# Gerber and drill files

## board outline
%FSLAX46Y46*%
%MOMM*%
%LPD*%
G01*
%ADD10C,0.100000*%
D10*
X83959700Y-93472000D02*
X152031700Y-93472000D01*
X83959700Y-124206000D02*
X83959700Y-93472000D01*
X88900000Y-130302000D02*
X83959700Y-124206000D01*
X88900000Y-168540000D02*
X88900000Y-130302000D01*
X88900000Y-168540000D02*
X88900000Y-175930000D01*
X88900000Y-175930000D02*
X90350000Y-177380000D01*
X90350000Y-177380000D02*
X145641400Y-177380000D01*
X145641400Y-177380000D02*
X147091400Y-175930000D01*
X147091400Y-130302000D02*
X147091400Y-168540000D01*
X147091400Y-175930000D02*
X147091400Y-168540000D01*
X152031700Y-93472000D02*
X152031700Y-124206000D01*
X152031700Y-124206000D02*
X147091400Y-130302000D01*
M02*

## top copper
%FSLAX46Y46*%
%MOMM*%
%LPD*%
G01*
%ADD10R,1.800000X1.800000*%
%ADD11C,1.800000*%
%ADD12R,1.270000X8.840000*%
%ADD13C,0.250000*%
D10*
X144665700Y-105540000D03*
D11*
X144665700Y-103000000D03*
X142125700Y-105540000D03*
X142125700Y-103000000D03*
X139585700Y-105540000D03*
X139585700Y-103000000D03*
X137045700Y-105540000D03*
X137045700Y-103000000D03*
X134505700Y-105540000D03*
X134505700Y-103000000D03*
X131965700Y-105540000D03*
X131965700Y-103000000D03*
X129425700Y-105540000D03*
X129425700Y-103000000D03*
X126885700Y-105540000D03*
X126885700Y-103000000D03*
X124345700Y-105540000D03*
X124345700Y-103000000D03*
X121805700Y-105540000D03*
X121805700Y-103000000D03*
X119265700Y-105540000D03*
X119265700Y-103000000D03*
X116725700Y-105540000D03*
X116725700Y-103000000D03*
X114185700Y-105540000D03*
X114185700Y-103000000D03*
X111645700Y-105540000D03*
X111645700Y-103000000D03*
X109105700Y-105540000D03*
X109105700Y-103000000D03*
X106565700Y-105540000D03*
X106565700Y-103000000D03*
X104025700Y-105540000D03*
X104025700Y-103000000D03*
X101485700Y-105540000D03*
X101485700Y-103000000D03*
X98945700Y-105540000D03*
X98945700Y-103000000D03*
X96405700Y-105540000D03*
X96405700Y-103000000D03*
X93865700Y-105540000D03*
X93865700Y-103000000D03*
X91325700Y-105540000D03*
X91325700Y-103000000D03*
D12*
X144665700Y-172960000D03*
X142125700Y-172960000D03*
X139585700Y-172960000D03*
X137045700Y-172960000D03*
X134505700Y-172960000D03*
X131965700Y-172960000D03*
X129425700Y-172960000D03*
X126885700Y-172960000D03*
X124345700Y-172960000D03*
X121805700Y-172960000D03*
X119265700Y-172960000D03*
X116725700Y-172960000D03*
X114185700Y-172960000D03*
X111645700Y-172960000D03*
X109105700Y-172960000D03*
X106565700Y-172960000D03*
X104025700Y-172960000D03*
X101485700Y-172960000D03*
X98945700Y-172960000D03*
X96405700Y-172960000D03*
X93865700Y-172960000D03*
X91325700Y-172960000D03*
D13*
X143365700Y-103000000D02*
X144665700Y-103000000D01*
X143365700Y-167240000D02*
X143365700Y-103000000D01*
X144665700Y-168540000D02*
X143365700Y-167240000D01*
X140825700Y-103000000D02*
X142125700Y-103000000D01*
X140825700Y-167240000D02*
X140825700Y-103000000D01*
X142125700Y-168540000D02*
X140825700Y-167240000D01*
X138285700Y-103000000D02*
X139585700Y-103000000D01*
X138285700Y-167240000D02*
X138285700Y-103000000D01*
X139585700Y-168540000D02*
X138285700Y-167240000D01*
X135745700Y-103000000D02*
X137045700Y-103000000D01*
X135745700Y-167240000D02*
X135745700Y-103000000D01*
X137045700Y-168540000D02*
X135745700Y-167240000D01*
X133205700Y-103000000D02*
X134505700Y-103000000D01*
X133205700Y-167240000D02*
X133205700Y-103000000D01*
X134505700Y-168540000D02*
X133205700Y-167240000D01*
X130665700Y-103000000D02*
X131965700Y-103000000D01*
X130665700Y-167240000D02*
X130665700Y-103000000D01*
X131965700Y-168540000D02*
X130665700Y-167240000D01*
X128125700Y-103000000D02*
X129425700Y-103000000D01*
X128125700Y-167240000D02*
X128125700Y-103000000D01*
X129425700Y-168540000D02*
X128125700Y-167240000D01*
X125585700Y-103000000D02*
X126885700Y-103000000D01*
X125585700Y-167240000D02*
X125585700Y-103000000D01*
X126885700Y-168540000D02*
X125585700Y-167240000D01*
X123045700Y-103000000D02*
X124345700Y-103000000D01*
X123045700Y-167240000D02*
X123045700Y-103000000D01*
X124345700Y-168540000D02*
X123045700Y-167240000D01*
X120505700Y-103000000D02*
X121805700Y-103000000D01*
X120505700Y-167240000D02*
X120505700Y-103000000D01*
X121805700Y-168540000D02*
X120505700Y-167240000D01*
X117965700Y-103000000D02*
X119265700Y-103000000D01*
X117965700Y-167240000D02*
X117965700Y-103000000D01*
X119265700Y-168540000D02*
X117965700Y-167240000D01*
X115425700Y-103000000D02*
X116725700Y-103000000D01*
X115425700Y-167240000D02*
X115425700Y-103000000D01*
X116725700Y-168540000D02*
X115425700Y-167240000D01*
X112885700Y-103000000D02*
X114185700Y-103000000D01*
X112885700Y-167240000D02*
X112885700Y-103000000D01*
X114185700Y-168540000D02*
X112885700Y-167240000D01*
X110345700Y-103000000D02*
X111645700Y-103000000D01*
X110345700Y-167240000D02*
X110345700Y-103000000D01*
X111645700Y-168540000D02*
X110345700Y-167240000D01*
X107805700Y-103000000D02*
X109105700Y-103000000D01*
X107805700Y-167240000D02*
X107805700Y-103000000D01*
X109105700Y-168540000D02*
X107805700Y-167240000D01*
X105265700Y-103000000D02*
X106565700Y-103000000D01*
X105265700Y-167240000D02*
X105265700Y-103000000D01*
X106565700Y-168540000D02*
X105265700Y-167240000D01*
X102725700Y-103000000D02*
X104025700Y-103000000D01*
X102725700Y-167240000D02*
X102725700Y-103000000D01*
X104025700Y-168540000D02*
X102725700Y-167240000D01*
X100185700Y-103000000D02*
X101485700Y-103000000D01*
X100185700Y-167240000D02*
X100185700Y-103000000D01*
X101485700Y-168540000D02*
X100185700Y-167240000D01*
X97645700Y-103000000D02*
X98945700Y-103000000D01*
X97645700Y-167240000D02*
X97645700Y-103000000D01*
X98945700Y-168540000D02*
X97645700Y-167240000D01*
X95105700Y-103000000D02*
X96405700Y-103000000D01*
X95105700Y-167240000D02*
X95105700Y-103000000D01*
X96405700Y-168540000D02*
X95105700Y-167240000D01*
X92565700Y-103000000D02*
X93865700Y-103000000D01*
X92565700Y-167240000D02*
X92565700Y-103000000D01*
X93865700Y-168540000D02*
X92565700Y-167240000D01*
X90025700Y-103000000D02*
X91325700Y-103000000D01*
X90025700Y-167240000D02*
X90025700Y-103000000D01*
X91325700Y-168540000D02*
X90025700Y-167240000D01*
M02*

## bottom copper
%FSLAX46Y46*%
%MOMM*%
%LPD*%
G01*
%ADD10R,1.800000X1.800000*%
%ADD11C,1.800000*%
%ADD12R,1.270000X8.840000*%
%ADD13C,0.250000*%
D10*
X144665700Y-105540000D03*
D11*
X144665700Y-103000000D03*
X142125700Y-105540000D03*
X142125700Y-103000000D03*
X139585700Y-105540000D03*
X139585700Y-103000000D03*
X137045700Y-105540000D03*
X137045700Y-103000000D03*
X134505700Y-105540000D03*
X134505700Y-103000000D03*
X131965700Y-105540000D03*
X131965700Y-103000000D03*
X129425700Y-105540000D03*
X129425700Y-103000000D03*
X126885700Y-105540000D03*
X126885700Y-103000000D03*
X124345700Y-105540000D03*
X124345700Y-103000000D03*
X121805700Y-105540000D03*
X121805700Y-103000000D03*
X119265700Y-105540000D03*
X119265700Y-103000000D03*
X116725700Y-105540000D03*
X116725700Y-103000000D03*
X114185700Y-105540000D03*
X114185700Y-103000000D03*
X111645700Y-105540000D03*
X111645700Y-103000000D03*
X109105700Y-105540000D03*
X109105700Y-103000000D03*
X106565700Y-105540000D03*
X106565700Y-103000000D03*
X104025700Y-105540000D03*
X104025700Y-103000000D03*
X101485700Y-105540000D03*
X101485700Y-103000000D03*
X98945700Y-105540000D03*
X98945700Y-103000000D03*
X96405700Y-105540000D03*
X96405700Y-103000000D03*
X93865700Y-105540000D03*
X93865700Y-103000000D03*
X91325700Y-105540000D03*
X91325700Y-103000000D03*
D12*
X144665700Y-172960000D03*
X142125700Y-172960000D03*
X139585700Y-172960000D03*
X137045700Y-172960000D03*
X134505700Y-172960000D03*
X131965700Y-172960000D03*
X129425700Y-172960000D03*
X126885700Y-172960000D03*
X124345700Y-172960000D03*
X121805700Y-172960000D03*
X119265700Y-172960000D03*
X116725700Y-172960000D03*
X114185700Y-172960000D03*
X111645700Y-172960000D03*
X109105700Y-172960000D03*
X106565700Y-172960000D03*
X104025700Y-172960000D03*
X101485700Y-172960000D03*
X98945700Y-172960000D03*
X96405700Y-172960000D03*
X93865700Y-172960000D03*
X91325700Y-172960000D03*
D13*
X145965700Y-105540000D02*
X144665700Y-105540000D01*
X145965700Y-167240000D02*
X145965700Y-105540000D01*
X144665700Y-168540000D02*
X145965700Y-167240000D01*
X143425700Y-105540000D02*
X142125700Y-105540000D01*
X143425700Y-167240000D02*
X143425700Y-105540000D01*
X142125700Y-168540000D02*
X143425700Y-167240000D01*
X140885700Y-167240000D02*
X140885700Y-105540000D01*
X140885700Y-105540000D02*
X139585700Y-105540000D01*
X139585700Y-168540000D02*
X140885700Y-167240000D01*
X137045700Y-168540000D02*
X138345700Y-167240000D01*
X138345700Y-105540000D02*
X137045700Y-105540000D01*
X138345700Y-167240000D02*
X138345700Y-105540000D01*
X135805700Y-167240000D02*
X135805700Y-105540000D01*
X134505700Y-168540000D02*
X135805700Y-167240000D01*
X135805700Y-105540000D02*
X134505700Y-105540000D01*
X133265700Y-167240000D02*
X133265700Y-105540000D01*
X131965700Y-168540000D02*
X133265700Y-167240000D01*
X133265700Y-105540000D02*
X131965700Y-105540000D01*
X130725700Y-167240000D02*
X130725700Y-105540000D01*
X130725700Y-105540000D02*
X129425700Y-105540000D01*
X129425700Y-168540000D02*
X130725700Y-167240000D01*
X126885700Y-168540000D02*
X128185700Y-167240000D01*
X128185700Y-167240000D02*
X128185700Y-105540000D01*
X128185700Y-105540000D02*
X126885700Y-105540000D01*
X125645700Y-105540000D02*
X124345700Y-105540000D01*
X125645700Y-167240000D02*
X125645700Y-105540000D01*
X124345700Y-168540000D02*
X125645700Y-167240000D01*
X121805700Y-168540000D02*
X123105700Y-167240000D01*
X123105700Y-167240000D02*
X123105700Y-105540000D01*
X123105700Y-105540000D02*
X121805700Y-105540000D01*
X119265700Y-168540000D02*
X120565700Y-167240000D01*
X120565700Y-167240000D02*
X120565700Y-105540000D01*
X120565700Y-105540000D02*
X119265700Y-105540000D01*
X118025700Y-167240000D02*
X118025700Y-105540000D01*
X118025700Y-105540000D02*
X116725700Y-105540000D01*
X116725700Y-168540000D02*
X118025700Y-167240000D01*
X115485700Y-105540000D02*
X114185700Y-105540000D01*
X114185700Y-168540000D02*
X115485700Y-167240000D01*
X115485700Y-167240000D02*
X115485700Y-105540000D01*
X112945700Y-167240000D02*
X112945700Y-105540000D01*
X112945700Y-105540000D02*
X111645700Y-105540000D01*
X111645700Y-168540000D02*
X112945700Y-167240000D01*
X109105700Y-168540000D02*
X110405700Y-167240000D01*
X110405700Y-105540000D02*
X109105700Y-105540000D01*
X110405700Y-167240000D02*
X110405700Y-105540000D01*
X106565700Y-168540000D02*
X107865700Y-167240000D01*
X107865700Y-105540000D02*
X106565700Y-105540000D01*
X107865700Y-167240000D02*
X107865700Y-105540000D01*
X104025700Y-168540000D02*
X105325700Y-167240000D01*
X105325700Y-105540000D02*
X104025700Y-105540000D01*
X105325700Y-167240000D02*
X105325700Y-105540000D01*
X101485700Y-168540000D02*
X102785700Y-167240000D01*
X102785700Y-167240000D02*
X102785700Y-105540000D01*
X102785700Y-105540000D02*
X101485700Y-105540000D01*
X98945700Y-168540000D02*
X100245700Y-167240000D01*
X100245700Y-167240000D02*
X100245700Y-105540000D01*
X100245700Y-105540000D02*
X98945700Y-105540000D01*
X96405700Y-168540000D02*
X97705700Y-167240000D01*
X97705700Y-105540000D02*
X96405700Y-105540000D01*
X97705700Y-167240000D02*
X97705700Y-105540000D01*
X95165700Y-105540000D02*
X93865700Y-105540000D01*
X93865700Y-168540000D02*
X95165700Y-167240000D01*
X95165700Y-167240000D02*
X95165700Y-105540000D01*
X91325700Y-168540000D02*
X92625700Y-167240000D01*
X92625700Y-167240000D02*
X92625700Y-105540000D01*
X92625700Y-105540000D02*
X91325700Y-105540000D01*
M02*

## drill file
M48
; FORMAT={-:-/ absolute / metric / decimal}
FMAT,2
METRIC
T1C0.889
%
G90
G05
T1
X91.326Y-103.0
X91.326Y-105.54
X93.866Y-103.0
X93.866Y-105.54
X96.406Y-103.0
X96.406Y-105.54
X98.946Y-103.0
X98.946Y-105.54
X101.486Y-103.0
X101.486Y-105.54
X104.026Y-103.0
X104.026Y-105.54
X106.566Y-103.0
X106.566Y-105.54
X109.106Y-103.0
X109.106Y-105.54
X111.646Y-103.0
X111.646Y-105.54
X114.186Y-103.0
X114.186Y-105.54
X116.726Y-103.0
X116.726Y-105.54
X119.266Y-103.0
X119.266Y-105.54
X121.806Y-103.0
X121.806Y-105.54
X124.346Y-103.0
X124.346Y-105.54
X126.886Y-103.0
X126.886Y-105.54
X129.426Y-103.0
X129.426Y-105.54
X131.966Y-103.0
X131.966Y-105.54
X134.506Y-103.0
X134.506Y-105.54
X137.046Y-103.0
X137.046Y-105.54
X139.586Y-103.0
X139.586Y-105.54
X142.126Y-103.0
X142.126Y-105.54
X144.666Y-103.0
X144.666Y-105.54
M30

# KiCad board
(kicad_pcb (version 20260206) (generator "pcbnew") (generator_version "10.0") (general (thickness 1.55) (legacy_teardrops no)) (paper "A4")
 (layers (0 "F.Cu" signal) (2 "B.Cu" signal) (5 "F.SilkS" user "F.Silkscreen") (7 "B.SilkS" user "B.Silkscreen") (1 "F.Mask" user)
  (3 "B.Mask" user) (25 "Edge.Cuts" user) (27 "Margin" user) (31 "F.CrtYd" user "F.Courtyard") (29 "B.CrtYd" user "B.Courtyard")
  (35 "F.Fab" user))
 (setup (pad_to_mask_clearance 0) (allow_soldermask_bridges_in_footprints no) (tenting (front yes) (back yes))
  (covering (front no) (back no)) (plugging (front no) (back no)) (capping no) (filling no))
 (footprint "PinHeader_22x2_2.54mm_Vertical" (layer "F.Cu") (at 0 0)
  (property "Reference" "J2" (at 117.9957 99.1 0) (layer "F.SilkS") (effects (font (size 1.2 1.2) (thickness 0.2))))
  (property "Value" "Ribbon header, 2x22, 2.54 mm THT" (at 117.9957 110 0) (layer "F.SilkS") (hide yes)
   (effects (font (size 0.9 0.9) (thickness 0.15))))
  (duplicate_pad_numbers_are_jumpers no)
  (pad "1" thru_hole rect (at 144.6657 105.54) (size 1.8 1.8) (drill 0.889) (layers "*.Cu" "*.Mask") (remove_unused_layers no)
   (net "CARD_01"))
  (pad "2" thru_hole circle (at 144.6657 103) (size 1.8 1.8) (drill 0.889) (layers "*.Cu" "*.Mask") (remove_unused_layers no)
   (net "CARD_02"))
  (pad "3" thru_hole circle (at 142.1257 105.54) (size 1.8 1.8) (drill 0.889) (layers "*.Cu" "*.Mask") (remove_unused_layers no)
   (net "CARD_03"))
  (pad "4" thru_hole circle (at 142.1257 103) (size 1.8 1.8) (drill 0.889) (layers "*.Cu" "*.Mask") (remove_unused_layers no)
   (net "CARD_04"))
  (pad "5" thru_hole circle (at 139.5857 105.54) (size 1.8 1.8) (drill 0.889) (layers "*.Cu" "*.Mask") (remove_unused_layers no)
   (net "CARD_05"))
  (pad "6" thru_hole circle (at 139.5857 103) (size 1.8 1.8) (drill 0.889) (layers "*.Cu" "*.Mask") (remove_unused_layers no)
   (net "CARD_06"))
  (pad "7" thru_hole circle (at 137.0457 105.54) (size 1.8 1.8) (drill 0.889) (layers "*.Cu" "*.Mask") (remove_unused_layers no)
   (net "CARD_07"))
  (pad "8" thru_hole circle (at 137.0457 103) (size 1.8 1.8) (drill 0.889) (layers "*.Cu" "*.Mask") (remove_unused_layers no)
   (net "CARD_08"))
  (pad "9" thru_hole circle (at 134.5057 105.54) (size 1.8 1.8) (drill 0.889) (layers "*.Cu" "*.Mask") (remove_unused_layers no)
   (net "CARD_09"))
  (pad "10" thru_hole circle (at 134.5057 103) (size 1.8 1.8) (drill 0.889) (layers "*.Cu" "*.Mask") (remove_unused_layers no)
   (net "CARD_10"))
  (pad "11" thru_hole circle (at 131.9657 105.54) (size 1.8 1.8) (drill 0.889) (layers "*.Cu" "*.Mask") (remove_unused_layers no)
   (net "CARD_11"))
  (pad "12" thru_hole circle (at 131.9657 103) (size 1.8 1.8) (drill 0.889) (layers "*.Cu" "*.Mask") (remove_unused_layers no)
   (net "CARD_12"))
  (pad "13" thru_hole circle (at 129.4257 105.54) (size 1.8 1.8) (drill 0.889) (layers "*.Cu" "*.Mask") (remove_unused_layers no)
   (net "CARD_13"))
  (pad "14" thru_hole circle (at 129.4257 103) (size 1.8 1.8) (drill 0.889) (layers "*.Cu" "*.Mask") (remove_unused_layers no)
   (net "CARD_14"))
  (pad "15" thru_hole circle (at 126.8857 105.54) (size 1.8 1.8) (drill 0.889) (layers "*.Cu" "*.Mask") (remove_unused_layers no)
   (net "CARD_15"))
  (pad "16" thru_hole circle (at 126.8857 103) (size 1.8 1.8) (drill 0.889) (layers "*.Cu" "*.Mask") (remove_unused_layers no)
   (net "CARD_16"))
  (pad "17" thru_hole circle (at 124.3457 105.54) (size 1.8 1.8) (drill 0.889) (layers "*.Cu" "*.Mask") (remove_unused_layers no)
   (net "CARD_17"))
  (pad "18" thru_hole circle (at 124.3457 103) (size 1.8 1.8) (drill 0.889) (layers "*.Cu" "*.Mask") (remove_unused_layers no)
   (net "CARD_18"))
  (pad "19" thru_hole circle (at 121.8057 105.54) (size 1.8 1.8) (drill 0.889) (layers "*.Cu" "*.Mask") (remove_unused_layers no)
   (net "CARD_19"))
  (pad "20" thru_hole circle (at 121.8057 103) (size 1.8 1.8) (drill 0.889) (layers "*.Cu" "*.Mask") (remove_unused_layers no)
   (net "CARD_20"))
  (pad "21" thru_hole circle (at 119.2657 105.54) (size 1.8 1.8) (drill 0.889) (layers "*.Cu" "*.Mask") (remove_unused_layers no)
   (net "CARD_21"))
  (pad "22" thru_hole circle (at 119.2657 103) (size 1.8 1.8) (drill 0.889) (layers "*.Cu" "*.Mask") (remove_unused_layers no)
   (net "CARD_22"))
  (pad "23" thru_hole circle (at 116.7257 105.54) (size 1.8 1.8) (drill 0.889) (layers "*.Cu" "*.Mask") (remove_unused_layers no)
   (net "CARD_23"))
  (pad "24" thru_hole circle (at 116.7257 103) (size 1.8 1.8) (drill 0.889) (layers "*.Cu" "*.Mask") (remove_unused_layers no)
   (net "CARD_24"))
  (pad "25" thru_hole circle (at 114.1857 105.54) (size 1.8 1.8) (drill 0.889) (layers "*.Cu" "*.Mask") (remove_unused_layers no)
   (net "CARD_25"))
  (pad "26" thru_hole circle (at 114.1857 103) (size 1.8 1.8) (drill 0.889) (layers "*.Cu" "*.Mask") (remove_unused_layers no)
   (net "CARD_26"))
  (pad "27" thru_hole circle (at 111.6457 105.54) (size 1.8 1.8) (drill 0.889) (layers "*.Cu" "*.Mask") (remove_unused_layers no)
   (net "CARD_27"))
  (pad "28" thru_hole circle (at 111.6457 103) (size 1.8 1.8) (drill 0.889) (layers "*.Cu" "*.Mask") (remove_unused_layers no)
   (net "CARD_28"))
  (pad "29" thru_hole circle (at 109.1057 105.54) (size 1.8 1.8) (drill 0.889) (layers "*.Cu" "*.Mask") (remove_unused_layers no)
   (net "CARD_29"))
  (pad "30" thru_hole circle (at 109.1057 103) (size 1.8 1.8) (drill 0.889) (layers "*.Cu" "*.Mask") (remove_unused_layers no)
   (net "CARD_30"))
  (pad "31" thru_hole circle (at 106.5657 105.54) (size 1.8 1.8) (drill 0.889) (layers "*.Cu" "*.Mask") (remove_unused_layers no)
   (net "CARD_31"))
  (pad "32" thru_hole circle (at 106.5657 103) (size 1.8 1.8) (drill 0.889) (layers "*.Cu" "*.Mask") (remove_unused_layers no)
   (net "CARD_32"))
  (pad "33" thru_hole circle (at 104.0257 105.54) (size 1.8 1.8) (drill 0.889) (layers "*.Cu" "*.Mask") (remove_unused_layers no)
   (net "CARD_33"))
  (pad "34" thru_hole circle (at 104.0257 103) (size 1.8 1.8) (drill 0.889) (layers "*.Cu" "*.Mask") (remove_unused_layers no)
   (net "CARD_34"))
  (pad "35" thru_hole circle (at 101.4857 105.54) (size 1.8 1.8) (drill 0.889) (layers "*.Cu" "*.Mask") (remove_unused_layers no)
   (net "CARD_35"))
  (pad "36" thru_hole circle (at 101.4857 103) (size 1.8 1.8) (drill 0.889) (layers "*.Cu" "*.Mask") (remove_unused_layers no)
   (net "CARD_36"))
  (pad "37" thru_hole circle (at 98.9457 105.54) (size 1.8 1.8) (drill 0.889) (layers "*.Cu" "*.Mask") (remove_unused_layers no)
   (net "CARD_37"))
  (pad "38" thru_hole circle (at 98.9457 103) (size 1.8 1.8) (drill 0.889) (layers "*.Cu" "*.Mask") (remove_unused_layers no)
   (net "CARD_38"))
  (pad "39" thru_hole circle (at 96.4057 105.54) (size 1.8 1.8) (drill 0.889) (layers "*.Cu" "*.Mask") (remove_unused_layers no)
   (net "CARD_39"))
  (pad "40" thru_hole circle (at 96.4057 103) (size 1.8 1.8) (drill 0.889) (layers "*.Cu" "*.Mask") (remove_unused_layers no)
   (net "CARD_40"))
  (pad "41" thru_hole circle (at 93.8657 105.54) (size 1.8 1.8) (drill 0.889) (layers "*.Cu" "*.Mask") (remove_unused_layers no)
   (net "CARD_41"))
  (pad "42" thru_hole circle (at 93.8657 103) (size 1.8 1.8) (drill 0.889) (layers "*.Cu" "*.Mask") (remove_unused_layers no)
   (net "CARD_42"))
  (pad "43" thru_hole circle (at 91.3257 105.54) (size 1.8 1.8) (drill 0.889) (layers "*.Cu" "*.Mask") (remove_unused_layers no)
   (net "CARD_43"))
  (pad "44" thru_hole circle (at 91.3257 103) (size 1.8 1.8) (drill 0.889) (layers "*.Cu" "*.Mask") (remove_unused_layers no)
   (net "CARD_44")))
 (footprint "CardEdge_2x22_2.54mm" (layer "F.Cu") (at 0 -15)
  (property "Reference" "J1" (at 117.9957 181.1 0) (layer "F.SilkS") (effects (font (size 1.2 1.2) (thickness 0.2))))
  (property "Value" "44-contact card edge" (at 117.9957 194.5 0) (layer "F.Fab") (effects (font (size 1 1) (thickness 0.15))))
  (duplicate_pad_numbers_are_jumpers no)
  (pad "1" connect rect (at 144.6657 187.96) (size 1.27 8.84) (layers "B.Cu" "B.Mask") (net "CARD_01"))
  (pad "2" connect rect (at 144.6657 187.96) (size 1.27 8.84) (layers "F.Cu" "F.Mask") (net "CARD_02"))
  (pad "3" connect rect (at 142.1257 187.96) (size 1.27 8.84) (layers "B.Cu" "B.Mask") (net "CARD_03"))
  (pad "4" connect rect (at 142.1257 187.96) (size 1.27 8.84) (layers "F.Cu" "F.Mask") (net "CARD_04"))
  (pad "5" connect rect (at 139.5857 187.96) (size 1.27 8.84) (layers "B.Cu" "B.Mask") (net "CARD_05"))
  (pad "6" connect rect (at 139.5857 187.96) (size 1.27 8.84) (layers "F.Cu" "F.Mask") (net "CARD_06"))
  (pad "7" connect rect (at 137.0457 187.96) (size 1.27 8.84) (layers "B.Cu" "B.Mask") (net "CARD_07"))
  (pad "8" connect rect (at 137.0457 187.96) (size 1.27 8.84) (layers "F.Cu" "F.Mask") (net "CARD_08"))
  (pad "9" connect rect (at 134.5057 187.96) (size 1.27 8.84) (layers "B.Cu" "B.Mask") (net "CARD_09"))
  (pad "10" connect rect (at 134.5057 187.96) (size 1.27 8.84) (layers "F.Cu" "F.Mask") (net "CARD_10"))
  (pad "11" connect rect (at 131.9657 187.96) (size 1.27 8.84) (layers "B.Cu" "B.Mask") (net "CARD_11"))
  (pad "12" connect rect (at 131.9657 187.96) (size 1.27 8.84) (layers "F.Cu" "F.Mask") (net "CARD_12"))
  (pad "13" connect rect (at 129.4257 187.96) (size 1.27 8.84) (layers "B.Cu" "B.Mask") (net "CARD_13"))
  (pad "14" connect rect (at 129.4257 187.96) (size 1.27 8.84) (layers "F.Cu" "F.Mask") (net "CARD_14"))
  (pad "15" connect rect (at 126.8857 187.96) (size 1.27 8.84) (layers "B.Cu" "B.Mask") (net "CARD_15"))
  (pad "16" connect rect (at 126.8857 187.96) (size 1.27 8.84) (layers "F.Cu" "F.Mask") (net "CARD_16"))
  (pad "17" connect rect (at 124.3457 187.96) (size 1.27 8.84) (layers "B.Cu" "B.Mask") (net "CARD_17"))
  (pad "18" connect rect (at 124.3457 187.96) (size 1.27 8.84) (layers "F.Cu" "F.Mask") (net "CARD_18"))
  (pad "19" connect rect (at 121.8057 187.96) (size 1.27 8.84) (layers "B.Cu" "B.Mask") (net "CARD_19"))
  (pad "20" connect rect (at 121.8057 187.96) (size 1.27 8.84) (layers "F.Cu" "F.Mask") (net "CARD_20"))
  (pad "21" connect rect (at 119.2657 187.96) (size 1.27 8.84) (layers "B.Cu" "B.Mask") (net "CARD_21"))
  (pad "22" connect rect (at 119.2657 187.96) (size 1.27 8.84) (layers "F.Cu" "F.Mask") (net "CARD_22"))
  (pad "23" connect rect (at 116.7257 187.96) (size 1.27 8.84) (layers "B.Cu" "B.Mask") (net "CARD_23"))
  (pad "24" connect rect (at 116.7257 187.96) (size 1.27 8.84) (layers "F.Cu" "F.Mask") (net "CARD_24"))
  (pad "25" connect rect (at 114.1857 187.96) (size 1.27 8.84) (layers "B.Cu" "B.Mask") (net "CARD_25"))
  (pad "26" connect rect (at 114.1857 187.96) (size 1.27 8.84) (layers "F.Cu" "F.Mask") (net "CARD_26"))
  (pad "27" connect rect (at 111.6457 187.96) (size 1.27 8.84) (layers "B.Cu" "B.Mask") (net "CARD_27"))
  (pad "28" connect rect (at 111.6457 187.96) (size 1.27 8.84) (layers "F.Cu" "F.Mask") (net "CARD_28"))
  (pad "29" connect rect (at 109.1057 187.96) (size 1.27 8.84) (layers "B.Cu" "B.Mask") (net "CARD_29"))
  (pad "30" connect rect (at 109.1057 187.96) (size 1.27 8.84) (layers "F.Cu" "F.Mask") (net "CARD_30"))
  (pad "31" connect rect (at 106.5657 187.96) (size 1.27 8.84) (layers "B.Cu" "B.Mask") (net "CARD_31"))
  (pad "32" connect rect (at 106.5657 187.96) (size 1.27 8.84) (layers "F.Cu" "F.Mask") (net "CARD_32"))
  (pad "33" connect rect (at 104.0257 187.96) (size 1.27 8.84) (layers "B.Cu" "B.Mask") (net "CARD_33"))
  (pad "34" connect rect (at 104.0257 187.96) (size 1.27 8.84) (layers "F.Cu" "F.Mask") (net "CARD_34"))
  (pad "35" connect rect (at 101.4857 187.96) (size 1.27 8.84) (layers "B.Cu" "B.Mask") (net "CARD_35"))
  (pad "36" connect rect (at 101.4857 187.96) (size 1.27 8.84) (layers "F.Cu" "F.Mask") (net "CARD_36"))
  (pad "37" connect rect (at 98.9457 187.96) (size 1.27 8.84) (layers "B.Cu" "B.Mask") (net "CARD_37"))
  (pad "38" connect rect (at 98.9457 187.96) (size 1.27 8.84) (layers "F.Cu" "F.Mask") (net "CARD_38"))
  (pad "39" connect rect (at 96.4057 187.96) (size 1.27 8.84) (layers "B.Cu" "B.Mask") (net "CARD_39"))
  (pad "40" connect rect (at 96.4057 187.96) (size 1.27 8.84) (layers "F.Cu" "F.Mask") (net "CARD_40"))
  (pad "41" connect rect (at 93.8657 187.96) (size 1.27 8.84) (layers "B.Cu" "B.Mask") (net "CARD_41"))
  (pad "42" connect rect (at 93.8657 187.96) (size 1.27 8.84) (layers "F.Cu" "F.Mask") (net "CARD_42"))
  (pad "43" connect rect (at 91.3257 187.96) (size 1.27 8.84) (layers "B.Cu" "B.Mask") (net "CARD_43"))
  (pad "44" connect rect (at 91.3257 187.96) (size 1.27 8.84) (layers "F.Cu" "F.Mask") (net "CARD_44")))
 (gr_line (start 83.9597 93.472) (end 152.0317 93.472) (stroke (width 0.1) (type solid)) (layer "Edge.Cuts"))
 (gr_line (start 83.9597 124.206) (end 83.9597 93.472) (stroke (width 0.1) (type solid)) (layer "Edge.Cuts"))
 (gr_line (start 88.9 130.302) (end 83.9597 124.206) (stroke (width 0.1) (type solid)) (layer "Edge.Cuts"))
 (gr_line (start 88.9 168.54) (end 88.9 130.302) (stroke (width 0.1) (type solid)) (layer "Edge.Cuts"))
 (gr_line (start 88.9 168.54) (end 88.9 175.93) (stroke (width 0.1) (type solid)) (layer "Edge.Cuts"))
 (gr_line (start 88.9 175.93) (end 90.35 177.38) (stroke (width 0.1) (type solid)) (layer "Edge.Cuts"))
 (gr_line (start 90.35 177.38) (end 145.6414 177.38) (stroke (width 0.1) (type solid)) (layer "Edge.Cuts"))
 (gr_line (start 145.6414 177.38) (end 147.0914 175.93) (stroke (width 0.1) (type solid)) (layer "Edge.Cuts"))
 (gr_line (start 147.0914 130.302) (end 147.0914 168.54) (stroke (width 0.1) (type solid)) (layer "Edge.Cuts"))
 (gr_line (start 147.0914 175.93) (end 147.0914 168.54) (stroke (width 0.1) (type solid)) (layer "Edge.Cuts"))
 (gr_line (start 152.0317 93.472) (end 152.0317 124.206) (stroke (width 0.1) (type solid)) (layer "Edge.Cuts"))
 (gr_line (start 152.0317 124.206) (end 147.0914 130.302) (stroke (width 0.1) (type solid)) (layer "Edge.Cuts"))
 (segment (start 145.9657 105.54) (end 144.6657 105.54) (width 0.25) (layer "B.Cu") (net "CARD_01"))
 (segment (start 145.9657 167.24) (end 145.9657 105.54) (width 0.25) (layer "B.Cu") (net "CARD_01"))
 (segment (start 144.6657 168.54) (end 145.9657 167.24) (width 0.25) (layer "B.Cu") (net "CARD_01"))
 (segment (start 143.3657 103) (end 144.6657 103) (width 0.25) (layer "F.Cu") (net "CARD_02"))
 (segment (start 143.3657 167.24) (end 143.3657 103) (width 0.25) (layer "F.Cu") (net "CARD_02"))
 (segment (start 144.6657 168.54) (end 143.3657 167.24) (width 0.25) (layer "F.Cu") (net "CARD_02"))
 (segment (start 143.4257 105.54) (end 142.1257 105.54) (width 0.25) (layer "B.Cu") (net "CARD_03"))
 (segment (start 143.4257 167.24) (end 143.4257 105.54) (width 0.25) (layer "B.Cu") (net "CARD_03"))
 (segment (start 142.1257 168.54) (end 143.4257 167.24) (width 0.25) (layer "B.Cu") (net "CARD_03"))
 (segment (start 140.8257 103) (end 142.1257 103) (width 0.25) (layer "F.Cu") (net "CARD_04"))
 (segment (start 140.8257 167.24) (end 140.8257 103) (width 0.25) (layer "F.Cu") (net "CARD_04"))
 (segment (start 142.1257 168.54) (end 140.8257 167.24) (width 0.25) (layer "F.Cu") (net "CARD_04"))
 (segment (start 140.8857 167.24) (end 140.8857 105.54) (width 0.25) (layer "B.Cu") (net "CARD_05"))
 (segment (start 140.8857 105.54) (end 139.5857 105.54) (width 0.25) (layer "B.Cu") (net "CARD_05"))
 (segment (start 139.5857 168.54) (end 140.8857 167.24) (width 0.25) (layer "B.Cu") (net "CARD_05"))
 (segment (start 138.2857 103) (end 139.5857 103) (width 0.25) (layer "F.Cu") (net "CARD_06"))
 (segment (start 138.2857 167.24) (end 138.2857 103) (width 0.25) (layer "F.Cu") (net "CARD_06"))
 (segment (start 139.5857 168.54) (end 138.2857 167.24) (width 0.25) (layer "F.Cu") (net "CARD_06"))
 (segment (start 137.0457 168.54) (end 138.3457 167.24) (width 0.25) (layer "B.Cu") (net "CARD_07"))
 (segment (start 138.3457 105.54) (end 137.0457 105.54) (width 0.25) (layer "B.Cu") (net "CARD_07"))
 (segment (start 138.3457 167.24) (end 138.3457 105.54) (width 0.25) (layer "B.Cu") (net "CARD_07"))
 (segment (start 135.7457 103) (end 137.0457 103) (width 0.25) (layer "F.Cu") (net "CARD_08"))
 (segment (start 135.7457 167.24) (end 135.7457 103) (width 0.25) (layer "F.Cu") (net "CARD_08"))
 (segment (start 137.0457 168.54) (end 135.7457 167.24) (width 0.25) (layer "F.Cu") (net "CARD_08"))
 (segment (start 135.8057 167.24) (end 135.8057 105.54) (width 0.25) (layer "B.Cu") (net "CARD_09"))
 (segment (start 134.5057 168.54) (end 135.8057 167.24) (width 0.25) (layer "B.Cu") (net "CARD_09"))
 (segment (start 135.8057 105.54) (end 134.5057 105.54) (width 0.25) (layer "B.Cu") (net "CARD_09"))
 (segment (start 133.2057 103) (end 134.5057 103) (width 0.25) (layer "F.Cu") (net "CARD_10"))
 (segment (start 133.2057 167.24) (end 133.2057 103) (width 0.25) (layer "F.Cu") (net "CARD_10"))
 (segment (start 134.5057 168.54) (end 133.2057 167.24) (width 0.25) (layer "F.Cu") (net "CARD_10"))
 (segment (start 133.2657 167.24) (end 133.2657 105.54) (width 0.25) (layer "B.Cu") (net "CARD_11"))
 (segment (start 131.9657 168.54) (end 133.2657 167.24) (width 0.25) (layer "B.Cu") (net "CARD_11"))
 (segment (start 133.2657 105.54) (end 131.9657 105.54) (width 0.25) (layer "B.Cu") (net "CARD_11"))
 (segment (start 130.6657 103) (end 131.9657 103) (width 0.25) (layer "F.Cu") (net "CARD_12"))
 (segment (start 130.6657 167.24) (end 130.6657 103) (width 0.25) (layer "F.Cu") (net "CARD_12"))
 (segment (start 131.9657 168.54) (end 130.6657 167.24) (width 0.25) (layer "F.Cu") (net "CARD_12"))
 (segment (start 130.7257 167.24) (end 130.7257 105.54) (width 0.25) (layer "B.Cu") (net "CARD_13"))
 (segment (start 130.7257 105.54) (end 129.4257 105.54) (width 0.25) (layer "B.Cu") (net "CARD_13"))
 (segment (start 129.4257 168.54) (end 130.7257 167.24) (width 0.25) (layer "B.Cu") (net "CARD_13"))
 (segment (start 128.1257 103) (end 129.4257 103) (width 0.25) (layer "F.Cu") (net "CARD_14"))
 (segment (start 128.1257 167.24) (end 128.1257 103) (width 0.25) (layer "F.Cu") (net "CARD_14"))
 (segment (start 129.4257 168.54) (end 128.1257 167.24) (width 0.25) (layer "F.Cu") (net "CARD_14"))
 (segment (start 126.8857 168.54) (end 128.1857 167.24) (width 0.25) (layer "B.Cu") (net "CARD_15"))
 (segment (start 128.1857 167.24) (end 128.1857 105.54) (width 0.25) (layer "B.Cu") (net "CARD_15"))
 (segment (start 128.1857 105.54) (end 126.8857 105.54) (width 0.25) (layer "B.Cu") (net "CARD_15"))
 (segment (start 125.5857 103) (end 126.8857 103) (width 0.25) (layer "F.Cu") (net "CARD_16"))
 (segment (start 125.5857 167.24) (end 125.5857 103) (width 0.25) (layer "F.Cu") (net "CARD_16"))
 (segment (start 126.8857 168.54) (end 125.5857 167.24) (width 0.25) (layer "F.Cu") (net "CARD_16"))
 (segment (start 125.6457 105.54) (end 124.3457 105.54) (width 0.25) (layer "B.Cu") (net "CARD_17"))
 (segment (start 125.6457 167.24) (end 125.6457 105.54) (width 0.25) (layer "B.Cu") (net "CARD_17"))
 (segment (start 124.3457 168.54) (end 125.6457 167.24) (width 0.25) (layer "B.Cu") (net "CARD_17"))
 (segment (start 123.0457 103) (end 124.3457 103) (width 0.25) (layer "F.Cu") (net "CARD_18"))
 (segment (start 123.0457 167.24) (end 123.0457 103) (width 0.25) (layer "F.Cu") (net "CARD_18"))
 (segment (start 124.3457 168.54) (end 123.0457 167.24) (width 0.25) (layer "F.Cu") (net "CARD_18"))
 (segment (start 121.8057 168.54) (end 123.1057 167.24) (width 0.25) (layer "B.Cu") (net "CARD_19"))
 (segment (start 123.1057 167.24) (end 123.1057 105.54) (width 0.25) (layer "B.Cu") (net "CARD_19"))
 (segment (start 123.1057 105.54) (end 121.8057 105.54) (width 0.25) (layer "B.Cu") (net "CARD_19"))
 (segment (start 120.5057 103) (end 121.8057 103) (width 0.25) (layer "F.Cu") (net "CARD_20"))
 (segment (start 120.5057 167.24) (end 120.5057 103) (width 0.25) (layer "F.Cu") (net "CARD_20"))
 (segment (start 121.8057 168.54) (end 120.5057 167.24) (width 0.25) (layer "F.Cu") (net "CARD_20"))
 (segment (start 119.2657 168.54) (end 120.5657 167.24) (width 0.25) (layer "B.Cu") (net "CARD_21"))
 (segment (start 120.5657 167.24) (end 120.5657 105.54) (width 0.25) (layer "B.Cu") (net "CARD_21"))
 (segment (start 120.5657 105.54) (end 119.2657 105.54) (width 0.25) (layer "B.Cu") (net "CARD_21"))
 (segment (start 117.9657 103) (end 119.2657 103) (width 0.25) (layer "F.Cu") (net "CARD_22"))
 (segment (start 117.9657 167.24) (end 117.9657 103) (width 0.25) (layer "F.Cu") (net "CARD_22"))
 (segment (start 119.2657 168.54) (end 117.9657 167.24) (width 0.25) (layer "F.Cu") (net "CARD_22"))
 (segment (start 118.0257 167.24) (end 118.0257 105.54) (width 0.25) (layer "B.Cu") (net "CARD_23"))
 (segment (start 118.0257 105.54) (end 116.7257 105.54) (width 0.25) (layer "B.Cu") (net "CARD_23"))
 (segment (start 116.7257 168.54) (end 118.0257 167.24) (width 0.25) (layer "B.Cu") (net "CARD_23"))
 (segment (start 115.4257 103) (end 116.7257 103) (width 0.25) (layer "F.Cu") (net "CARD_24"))
 (segment (start 115.4257 167.24) (end 115.4257 103) (width 0.25) (layer "F.Cu") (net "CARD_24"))
 (segment (start 116.7257 168.54) (end 115.4257 167.24) (width 0.25) (layer "F.Cu") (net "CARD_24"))
 (segment (start 115.4857 105.54) (end 114.1857 105.54) (width 0.25) (layer "B.Cu") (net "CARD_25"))
 (segment (start 114.1857 168.54) (end 115.4857 167.24) (width 0.25) (layer "B.Cu") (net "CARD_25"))
 (segment (start 115.4857 167.24) (end 115.4857 105.54) (width 0.25) (layer "B.Cu") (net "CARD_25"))
 (segment (start 112.8857 103) (end 114.1857 103) (width 0.25) (layer "F.Cu") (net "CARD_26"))
 (segment (start 112.8857 167.24) (end 112.8857 103) (width 0.25) (layer "F.Cu") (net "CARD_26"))
 (segment (start 114.1857 168.54) (end 112.8857 167.24) (width 0.25) (layer "F.Cu") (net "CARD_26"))
 (segment (start 112.9457 167.24) (end 112.9457 105.54) (width 0.25) (layer "B.Cu") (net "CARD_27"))
 (segment (start 112.9457 105.54) (end 111.6457 105.54) (width 0.25) (layer "B.Cu") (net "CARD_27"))
 (segment (start 111.6457 168.54) (end 112.9457 167.24) (width 0.25) (layer "B.Cu") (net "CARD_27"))
 (segment (start 110.3457 103) (end 111.6457 103) (width 0.25) (layer "F.Cu") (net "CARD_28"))
 (segment (start 110.3457 167.24) (end 110.3457 103) (width 0.25) (layer "F.Cu") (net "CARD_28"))
 (segment (start 111.6457 168.54) (end 110.3457 167.24) (width 0.25) (layer "F.Cu") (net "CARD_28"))
 (segment (start 109.1057 168.54) (end 110.4057 167.24) (width 0.25) (layer "B.Cu") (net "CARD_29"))
 (segment (start 110.4057 105.54) (end 109.1057 105.54) (width 0.25) (layer "B.Cu") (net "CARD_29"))
 (segment (start 110.4057 167.24) (end 110.4057 105.54) (width 0.25) (layer "B.Cu") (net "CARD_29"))
 (segment (start 107.8057 103) (end 109.1057 103) (width 0.25) (layer "F.Cu") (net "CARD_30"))
 (segment (start 107.8057 167.24) (end 107.8057 103) (width 0.25) (layer "F.Cu") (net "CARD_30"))
 (segment (start 109.1057 168.54) (end 107.8057 167.24) (width 0.25) (layer "F.Cu") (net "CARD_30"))
 (segment (start 106.5657 168.54) (end 107.8657 167.24) (width 0.25) (layer "B.Cu") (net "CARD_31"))
 (segment (start 107.8657 105.54) (end 106.5657 105.54) (width 0.25) (layer "B.Cu") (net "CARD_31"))
 (segment (start 107.8657 167.24) (end 107.8657 105.54) (width 0.25) (layer "B.Cu") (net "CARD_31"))
 (segment (start 105.2657 103) (end 106.5657 103) (width 0.25) (layer "F.Cu") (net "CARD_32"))
 (segment (start 105.2657 167.24) (end 105.2657 103) (width 0.25) (layer "F.Cu") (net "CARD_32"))
 (segment (start 106.5657 168.54) (end 105.2657 167.24) (width 0.25) (layer "F.Cu") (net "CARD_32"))
 (segment (start 104.0257 168.54) (end 105.3257 167.24) (width 0.25) (layer "B.Cu") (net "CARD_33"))
 (segment (start 105.3257 105.54) (end 104.0257 105.54) (width 0.25) (layer "B.Cu") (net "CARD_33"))
 (segment (start 105.3257 167.24) (end 105.3257 105.54) (width 0.25) (layer "B.Cu") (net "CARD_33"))
 (segment (start 102.7257 103) (end 104.0257 103) (width 0.25) (layer "F.Cu") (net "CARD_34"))
 (segment (start 102.7257 167.24) (end 102.7257 103) (width 0.25) (layer "F.Cu") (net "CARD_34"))
 (segment (start 104.0257 168.54) (end 102.7257 167.24) (width 0.25) (layer "F.Cu") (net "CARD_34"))
 (segment (start 101.4857 168.54) (end 102.7857 167.24) (width 0.25) (layer "B.Cu") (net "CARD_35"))
 (segment (start 102.7857 167.24) (end 102.7857 105.54) (width 0.25) (layer "B.Cu") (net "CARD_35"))
 (segment (start 102.7857 105.54) (end 101.4857 105.54) (width 0.25) (layer "B.Cu") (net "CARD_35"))
 (segment (start 100.1857 103) (end 101.4857 103) (width 0.25) (layer "F.Cu") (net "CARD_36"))
 (segment (start 100.1857 167.24) (end 100.1857 103) (width 0.25) (layer "F.Cu") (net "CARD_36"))
 (segment (start 101.4857 168.54) (end 100.1857 167.24) (width 0.25) (layer "F.Cu") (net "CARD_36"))
 (segment (start 98.9457 168.54) (end 100.2457 167.24) (width 0.25) (layer "B.Cu") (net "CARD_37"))
 (segment (start 100.2457 167.24) (end 100.2457 105.54) (width 0.25) (layer "B.Cu") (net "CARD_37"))
 (segment (start 100.2457 105.54) (end 98.9457 105.54) (width 0.25) (layer "B.Cu") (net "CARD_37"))
 (segment (start 97.6457 103) (end 98.9457 103) (width 0.25) (layer "F.Cu") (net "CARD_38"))
 (segment (start 97.6457 167.24) (end 97.6457 103) (width 0.25) (layer "F.Cu") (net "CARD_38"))
 (segment (start 98.9457 168.54) (end 97.6457 167.24) (width 0.25) (layer "F.Cu") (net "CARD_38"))
 (segment (start 96.4057 168.54) (end 97.7057 167.24) (width 0.25) (layer "B.Cu") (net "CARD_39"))
 (segment (start 97.7057 105.54) (end 96.4057 105.54) (width 0.25) (layer "B.Cu") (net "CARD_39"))
 (segment (start 97.7057 167.24) (end 97.7057 105.54) (width 0.25) (layer "B.Cu") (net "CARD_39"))
 (segment (start 95.1057 103) (end 96.4057 103) (width 0.25) (layer "F.Cu") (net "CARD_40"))
 (segment (start 95.1057 167.24) (end 95.1057 103) (width 0.25) (layer "F.Cu") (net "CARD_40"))
 (segment (start 96.4057 168.54) (end 95.1057 167.24) (width 0.25) (layer "F.Cu") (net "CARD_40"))
 (segment (start 95.1657 105.54) (end 93.8657 105.54) (width 0.25) (layer "B.Cu") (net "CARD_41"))
 (segment (start 93.8657 168.54) (end 95.1657 167.24) (width 0.25) (layer "B.Cu") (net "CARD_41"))
 (segment (start 95.1657 167.24) (end 95.1657 105.54) (width 0.25) (layer "B.Cu") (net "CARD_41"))
 (segment (start 92.5657 103) (end 93.8657 103) (width 0.25) (layer "F.Cu") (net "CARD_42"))
 (segment (start 92.5657 167.24) (end 92.5657 103) (width 0.25) (layer "F.Cu") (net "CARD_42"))
 (segment (start 93.8657 168.54) (end 92.5657 167.24) (width 0.25) (layer "F.Cu") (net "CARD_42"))
 (segment (start 91.3257 168.54) (end 92.6257 167.24) (width 0.25) (layer "B.Cu") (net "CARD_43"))
 (segment (start 92.6257 167.24) (end 92.6257 105.54) (width 0.25) (layer "B.Cu") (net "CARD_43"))
 (segment (start 92.6257 105.54) (end 91.3257 105.54) (width 0.25) (layer "B.Cu") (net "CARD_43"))
 (segment (start 90.0257 103) (end 91.3257 103) (width 0.25) (layer "F.Cu") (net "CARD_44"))
 (segment (start 90.0257 167.24) (end 90.0257 103) (width 0.25) (layer "F.Cu") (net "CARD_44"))
 (segment (start 91.3257 168.54) (end 90.0257 167.24) (width 0.25) (layer "F.Cu") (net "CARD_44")))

